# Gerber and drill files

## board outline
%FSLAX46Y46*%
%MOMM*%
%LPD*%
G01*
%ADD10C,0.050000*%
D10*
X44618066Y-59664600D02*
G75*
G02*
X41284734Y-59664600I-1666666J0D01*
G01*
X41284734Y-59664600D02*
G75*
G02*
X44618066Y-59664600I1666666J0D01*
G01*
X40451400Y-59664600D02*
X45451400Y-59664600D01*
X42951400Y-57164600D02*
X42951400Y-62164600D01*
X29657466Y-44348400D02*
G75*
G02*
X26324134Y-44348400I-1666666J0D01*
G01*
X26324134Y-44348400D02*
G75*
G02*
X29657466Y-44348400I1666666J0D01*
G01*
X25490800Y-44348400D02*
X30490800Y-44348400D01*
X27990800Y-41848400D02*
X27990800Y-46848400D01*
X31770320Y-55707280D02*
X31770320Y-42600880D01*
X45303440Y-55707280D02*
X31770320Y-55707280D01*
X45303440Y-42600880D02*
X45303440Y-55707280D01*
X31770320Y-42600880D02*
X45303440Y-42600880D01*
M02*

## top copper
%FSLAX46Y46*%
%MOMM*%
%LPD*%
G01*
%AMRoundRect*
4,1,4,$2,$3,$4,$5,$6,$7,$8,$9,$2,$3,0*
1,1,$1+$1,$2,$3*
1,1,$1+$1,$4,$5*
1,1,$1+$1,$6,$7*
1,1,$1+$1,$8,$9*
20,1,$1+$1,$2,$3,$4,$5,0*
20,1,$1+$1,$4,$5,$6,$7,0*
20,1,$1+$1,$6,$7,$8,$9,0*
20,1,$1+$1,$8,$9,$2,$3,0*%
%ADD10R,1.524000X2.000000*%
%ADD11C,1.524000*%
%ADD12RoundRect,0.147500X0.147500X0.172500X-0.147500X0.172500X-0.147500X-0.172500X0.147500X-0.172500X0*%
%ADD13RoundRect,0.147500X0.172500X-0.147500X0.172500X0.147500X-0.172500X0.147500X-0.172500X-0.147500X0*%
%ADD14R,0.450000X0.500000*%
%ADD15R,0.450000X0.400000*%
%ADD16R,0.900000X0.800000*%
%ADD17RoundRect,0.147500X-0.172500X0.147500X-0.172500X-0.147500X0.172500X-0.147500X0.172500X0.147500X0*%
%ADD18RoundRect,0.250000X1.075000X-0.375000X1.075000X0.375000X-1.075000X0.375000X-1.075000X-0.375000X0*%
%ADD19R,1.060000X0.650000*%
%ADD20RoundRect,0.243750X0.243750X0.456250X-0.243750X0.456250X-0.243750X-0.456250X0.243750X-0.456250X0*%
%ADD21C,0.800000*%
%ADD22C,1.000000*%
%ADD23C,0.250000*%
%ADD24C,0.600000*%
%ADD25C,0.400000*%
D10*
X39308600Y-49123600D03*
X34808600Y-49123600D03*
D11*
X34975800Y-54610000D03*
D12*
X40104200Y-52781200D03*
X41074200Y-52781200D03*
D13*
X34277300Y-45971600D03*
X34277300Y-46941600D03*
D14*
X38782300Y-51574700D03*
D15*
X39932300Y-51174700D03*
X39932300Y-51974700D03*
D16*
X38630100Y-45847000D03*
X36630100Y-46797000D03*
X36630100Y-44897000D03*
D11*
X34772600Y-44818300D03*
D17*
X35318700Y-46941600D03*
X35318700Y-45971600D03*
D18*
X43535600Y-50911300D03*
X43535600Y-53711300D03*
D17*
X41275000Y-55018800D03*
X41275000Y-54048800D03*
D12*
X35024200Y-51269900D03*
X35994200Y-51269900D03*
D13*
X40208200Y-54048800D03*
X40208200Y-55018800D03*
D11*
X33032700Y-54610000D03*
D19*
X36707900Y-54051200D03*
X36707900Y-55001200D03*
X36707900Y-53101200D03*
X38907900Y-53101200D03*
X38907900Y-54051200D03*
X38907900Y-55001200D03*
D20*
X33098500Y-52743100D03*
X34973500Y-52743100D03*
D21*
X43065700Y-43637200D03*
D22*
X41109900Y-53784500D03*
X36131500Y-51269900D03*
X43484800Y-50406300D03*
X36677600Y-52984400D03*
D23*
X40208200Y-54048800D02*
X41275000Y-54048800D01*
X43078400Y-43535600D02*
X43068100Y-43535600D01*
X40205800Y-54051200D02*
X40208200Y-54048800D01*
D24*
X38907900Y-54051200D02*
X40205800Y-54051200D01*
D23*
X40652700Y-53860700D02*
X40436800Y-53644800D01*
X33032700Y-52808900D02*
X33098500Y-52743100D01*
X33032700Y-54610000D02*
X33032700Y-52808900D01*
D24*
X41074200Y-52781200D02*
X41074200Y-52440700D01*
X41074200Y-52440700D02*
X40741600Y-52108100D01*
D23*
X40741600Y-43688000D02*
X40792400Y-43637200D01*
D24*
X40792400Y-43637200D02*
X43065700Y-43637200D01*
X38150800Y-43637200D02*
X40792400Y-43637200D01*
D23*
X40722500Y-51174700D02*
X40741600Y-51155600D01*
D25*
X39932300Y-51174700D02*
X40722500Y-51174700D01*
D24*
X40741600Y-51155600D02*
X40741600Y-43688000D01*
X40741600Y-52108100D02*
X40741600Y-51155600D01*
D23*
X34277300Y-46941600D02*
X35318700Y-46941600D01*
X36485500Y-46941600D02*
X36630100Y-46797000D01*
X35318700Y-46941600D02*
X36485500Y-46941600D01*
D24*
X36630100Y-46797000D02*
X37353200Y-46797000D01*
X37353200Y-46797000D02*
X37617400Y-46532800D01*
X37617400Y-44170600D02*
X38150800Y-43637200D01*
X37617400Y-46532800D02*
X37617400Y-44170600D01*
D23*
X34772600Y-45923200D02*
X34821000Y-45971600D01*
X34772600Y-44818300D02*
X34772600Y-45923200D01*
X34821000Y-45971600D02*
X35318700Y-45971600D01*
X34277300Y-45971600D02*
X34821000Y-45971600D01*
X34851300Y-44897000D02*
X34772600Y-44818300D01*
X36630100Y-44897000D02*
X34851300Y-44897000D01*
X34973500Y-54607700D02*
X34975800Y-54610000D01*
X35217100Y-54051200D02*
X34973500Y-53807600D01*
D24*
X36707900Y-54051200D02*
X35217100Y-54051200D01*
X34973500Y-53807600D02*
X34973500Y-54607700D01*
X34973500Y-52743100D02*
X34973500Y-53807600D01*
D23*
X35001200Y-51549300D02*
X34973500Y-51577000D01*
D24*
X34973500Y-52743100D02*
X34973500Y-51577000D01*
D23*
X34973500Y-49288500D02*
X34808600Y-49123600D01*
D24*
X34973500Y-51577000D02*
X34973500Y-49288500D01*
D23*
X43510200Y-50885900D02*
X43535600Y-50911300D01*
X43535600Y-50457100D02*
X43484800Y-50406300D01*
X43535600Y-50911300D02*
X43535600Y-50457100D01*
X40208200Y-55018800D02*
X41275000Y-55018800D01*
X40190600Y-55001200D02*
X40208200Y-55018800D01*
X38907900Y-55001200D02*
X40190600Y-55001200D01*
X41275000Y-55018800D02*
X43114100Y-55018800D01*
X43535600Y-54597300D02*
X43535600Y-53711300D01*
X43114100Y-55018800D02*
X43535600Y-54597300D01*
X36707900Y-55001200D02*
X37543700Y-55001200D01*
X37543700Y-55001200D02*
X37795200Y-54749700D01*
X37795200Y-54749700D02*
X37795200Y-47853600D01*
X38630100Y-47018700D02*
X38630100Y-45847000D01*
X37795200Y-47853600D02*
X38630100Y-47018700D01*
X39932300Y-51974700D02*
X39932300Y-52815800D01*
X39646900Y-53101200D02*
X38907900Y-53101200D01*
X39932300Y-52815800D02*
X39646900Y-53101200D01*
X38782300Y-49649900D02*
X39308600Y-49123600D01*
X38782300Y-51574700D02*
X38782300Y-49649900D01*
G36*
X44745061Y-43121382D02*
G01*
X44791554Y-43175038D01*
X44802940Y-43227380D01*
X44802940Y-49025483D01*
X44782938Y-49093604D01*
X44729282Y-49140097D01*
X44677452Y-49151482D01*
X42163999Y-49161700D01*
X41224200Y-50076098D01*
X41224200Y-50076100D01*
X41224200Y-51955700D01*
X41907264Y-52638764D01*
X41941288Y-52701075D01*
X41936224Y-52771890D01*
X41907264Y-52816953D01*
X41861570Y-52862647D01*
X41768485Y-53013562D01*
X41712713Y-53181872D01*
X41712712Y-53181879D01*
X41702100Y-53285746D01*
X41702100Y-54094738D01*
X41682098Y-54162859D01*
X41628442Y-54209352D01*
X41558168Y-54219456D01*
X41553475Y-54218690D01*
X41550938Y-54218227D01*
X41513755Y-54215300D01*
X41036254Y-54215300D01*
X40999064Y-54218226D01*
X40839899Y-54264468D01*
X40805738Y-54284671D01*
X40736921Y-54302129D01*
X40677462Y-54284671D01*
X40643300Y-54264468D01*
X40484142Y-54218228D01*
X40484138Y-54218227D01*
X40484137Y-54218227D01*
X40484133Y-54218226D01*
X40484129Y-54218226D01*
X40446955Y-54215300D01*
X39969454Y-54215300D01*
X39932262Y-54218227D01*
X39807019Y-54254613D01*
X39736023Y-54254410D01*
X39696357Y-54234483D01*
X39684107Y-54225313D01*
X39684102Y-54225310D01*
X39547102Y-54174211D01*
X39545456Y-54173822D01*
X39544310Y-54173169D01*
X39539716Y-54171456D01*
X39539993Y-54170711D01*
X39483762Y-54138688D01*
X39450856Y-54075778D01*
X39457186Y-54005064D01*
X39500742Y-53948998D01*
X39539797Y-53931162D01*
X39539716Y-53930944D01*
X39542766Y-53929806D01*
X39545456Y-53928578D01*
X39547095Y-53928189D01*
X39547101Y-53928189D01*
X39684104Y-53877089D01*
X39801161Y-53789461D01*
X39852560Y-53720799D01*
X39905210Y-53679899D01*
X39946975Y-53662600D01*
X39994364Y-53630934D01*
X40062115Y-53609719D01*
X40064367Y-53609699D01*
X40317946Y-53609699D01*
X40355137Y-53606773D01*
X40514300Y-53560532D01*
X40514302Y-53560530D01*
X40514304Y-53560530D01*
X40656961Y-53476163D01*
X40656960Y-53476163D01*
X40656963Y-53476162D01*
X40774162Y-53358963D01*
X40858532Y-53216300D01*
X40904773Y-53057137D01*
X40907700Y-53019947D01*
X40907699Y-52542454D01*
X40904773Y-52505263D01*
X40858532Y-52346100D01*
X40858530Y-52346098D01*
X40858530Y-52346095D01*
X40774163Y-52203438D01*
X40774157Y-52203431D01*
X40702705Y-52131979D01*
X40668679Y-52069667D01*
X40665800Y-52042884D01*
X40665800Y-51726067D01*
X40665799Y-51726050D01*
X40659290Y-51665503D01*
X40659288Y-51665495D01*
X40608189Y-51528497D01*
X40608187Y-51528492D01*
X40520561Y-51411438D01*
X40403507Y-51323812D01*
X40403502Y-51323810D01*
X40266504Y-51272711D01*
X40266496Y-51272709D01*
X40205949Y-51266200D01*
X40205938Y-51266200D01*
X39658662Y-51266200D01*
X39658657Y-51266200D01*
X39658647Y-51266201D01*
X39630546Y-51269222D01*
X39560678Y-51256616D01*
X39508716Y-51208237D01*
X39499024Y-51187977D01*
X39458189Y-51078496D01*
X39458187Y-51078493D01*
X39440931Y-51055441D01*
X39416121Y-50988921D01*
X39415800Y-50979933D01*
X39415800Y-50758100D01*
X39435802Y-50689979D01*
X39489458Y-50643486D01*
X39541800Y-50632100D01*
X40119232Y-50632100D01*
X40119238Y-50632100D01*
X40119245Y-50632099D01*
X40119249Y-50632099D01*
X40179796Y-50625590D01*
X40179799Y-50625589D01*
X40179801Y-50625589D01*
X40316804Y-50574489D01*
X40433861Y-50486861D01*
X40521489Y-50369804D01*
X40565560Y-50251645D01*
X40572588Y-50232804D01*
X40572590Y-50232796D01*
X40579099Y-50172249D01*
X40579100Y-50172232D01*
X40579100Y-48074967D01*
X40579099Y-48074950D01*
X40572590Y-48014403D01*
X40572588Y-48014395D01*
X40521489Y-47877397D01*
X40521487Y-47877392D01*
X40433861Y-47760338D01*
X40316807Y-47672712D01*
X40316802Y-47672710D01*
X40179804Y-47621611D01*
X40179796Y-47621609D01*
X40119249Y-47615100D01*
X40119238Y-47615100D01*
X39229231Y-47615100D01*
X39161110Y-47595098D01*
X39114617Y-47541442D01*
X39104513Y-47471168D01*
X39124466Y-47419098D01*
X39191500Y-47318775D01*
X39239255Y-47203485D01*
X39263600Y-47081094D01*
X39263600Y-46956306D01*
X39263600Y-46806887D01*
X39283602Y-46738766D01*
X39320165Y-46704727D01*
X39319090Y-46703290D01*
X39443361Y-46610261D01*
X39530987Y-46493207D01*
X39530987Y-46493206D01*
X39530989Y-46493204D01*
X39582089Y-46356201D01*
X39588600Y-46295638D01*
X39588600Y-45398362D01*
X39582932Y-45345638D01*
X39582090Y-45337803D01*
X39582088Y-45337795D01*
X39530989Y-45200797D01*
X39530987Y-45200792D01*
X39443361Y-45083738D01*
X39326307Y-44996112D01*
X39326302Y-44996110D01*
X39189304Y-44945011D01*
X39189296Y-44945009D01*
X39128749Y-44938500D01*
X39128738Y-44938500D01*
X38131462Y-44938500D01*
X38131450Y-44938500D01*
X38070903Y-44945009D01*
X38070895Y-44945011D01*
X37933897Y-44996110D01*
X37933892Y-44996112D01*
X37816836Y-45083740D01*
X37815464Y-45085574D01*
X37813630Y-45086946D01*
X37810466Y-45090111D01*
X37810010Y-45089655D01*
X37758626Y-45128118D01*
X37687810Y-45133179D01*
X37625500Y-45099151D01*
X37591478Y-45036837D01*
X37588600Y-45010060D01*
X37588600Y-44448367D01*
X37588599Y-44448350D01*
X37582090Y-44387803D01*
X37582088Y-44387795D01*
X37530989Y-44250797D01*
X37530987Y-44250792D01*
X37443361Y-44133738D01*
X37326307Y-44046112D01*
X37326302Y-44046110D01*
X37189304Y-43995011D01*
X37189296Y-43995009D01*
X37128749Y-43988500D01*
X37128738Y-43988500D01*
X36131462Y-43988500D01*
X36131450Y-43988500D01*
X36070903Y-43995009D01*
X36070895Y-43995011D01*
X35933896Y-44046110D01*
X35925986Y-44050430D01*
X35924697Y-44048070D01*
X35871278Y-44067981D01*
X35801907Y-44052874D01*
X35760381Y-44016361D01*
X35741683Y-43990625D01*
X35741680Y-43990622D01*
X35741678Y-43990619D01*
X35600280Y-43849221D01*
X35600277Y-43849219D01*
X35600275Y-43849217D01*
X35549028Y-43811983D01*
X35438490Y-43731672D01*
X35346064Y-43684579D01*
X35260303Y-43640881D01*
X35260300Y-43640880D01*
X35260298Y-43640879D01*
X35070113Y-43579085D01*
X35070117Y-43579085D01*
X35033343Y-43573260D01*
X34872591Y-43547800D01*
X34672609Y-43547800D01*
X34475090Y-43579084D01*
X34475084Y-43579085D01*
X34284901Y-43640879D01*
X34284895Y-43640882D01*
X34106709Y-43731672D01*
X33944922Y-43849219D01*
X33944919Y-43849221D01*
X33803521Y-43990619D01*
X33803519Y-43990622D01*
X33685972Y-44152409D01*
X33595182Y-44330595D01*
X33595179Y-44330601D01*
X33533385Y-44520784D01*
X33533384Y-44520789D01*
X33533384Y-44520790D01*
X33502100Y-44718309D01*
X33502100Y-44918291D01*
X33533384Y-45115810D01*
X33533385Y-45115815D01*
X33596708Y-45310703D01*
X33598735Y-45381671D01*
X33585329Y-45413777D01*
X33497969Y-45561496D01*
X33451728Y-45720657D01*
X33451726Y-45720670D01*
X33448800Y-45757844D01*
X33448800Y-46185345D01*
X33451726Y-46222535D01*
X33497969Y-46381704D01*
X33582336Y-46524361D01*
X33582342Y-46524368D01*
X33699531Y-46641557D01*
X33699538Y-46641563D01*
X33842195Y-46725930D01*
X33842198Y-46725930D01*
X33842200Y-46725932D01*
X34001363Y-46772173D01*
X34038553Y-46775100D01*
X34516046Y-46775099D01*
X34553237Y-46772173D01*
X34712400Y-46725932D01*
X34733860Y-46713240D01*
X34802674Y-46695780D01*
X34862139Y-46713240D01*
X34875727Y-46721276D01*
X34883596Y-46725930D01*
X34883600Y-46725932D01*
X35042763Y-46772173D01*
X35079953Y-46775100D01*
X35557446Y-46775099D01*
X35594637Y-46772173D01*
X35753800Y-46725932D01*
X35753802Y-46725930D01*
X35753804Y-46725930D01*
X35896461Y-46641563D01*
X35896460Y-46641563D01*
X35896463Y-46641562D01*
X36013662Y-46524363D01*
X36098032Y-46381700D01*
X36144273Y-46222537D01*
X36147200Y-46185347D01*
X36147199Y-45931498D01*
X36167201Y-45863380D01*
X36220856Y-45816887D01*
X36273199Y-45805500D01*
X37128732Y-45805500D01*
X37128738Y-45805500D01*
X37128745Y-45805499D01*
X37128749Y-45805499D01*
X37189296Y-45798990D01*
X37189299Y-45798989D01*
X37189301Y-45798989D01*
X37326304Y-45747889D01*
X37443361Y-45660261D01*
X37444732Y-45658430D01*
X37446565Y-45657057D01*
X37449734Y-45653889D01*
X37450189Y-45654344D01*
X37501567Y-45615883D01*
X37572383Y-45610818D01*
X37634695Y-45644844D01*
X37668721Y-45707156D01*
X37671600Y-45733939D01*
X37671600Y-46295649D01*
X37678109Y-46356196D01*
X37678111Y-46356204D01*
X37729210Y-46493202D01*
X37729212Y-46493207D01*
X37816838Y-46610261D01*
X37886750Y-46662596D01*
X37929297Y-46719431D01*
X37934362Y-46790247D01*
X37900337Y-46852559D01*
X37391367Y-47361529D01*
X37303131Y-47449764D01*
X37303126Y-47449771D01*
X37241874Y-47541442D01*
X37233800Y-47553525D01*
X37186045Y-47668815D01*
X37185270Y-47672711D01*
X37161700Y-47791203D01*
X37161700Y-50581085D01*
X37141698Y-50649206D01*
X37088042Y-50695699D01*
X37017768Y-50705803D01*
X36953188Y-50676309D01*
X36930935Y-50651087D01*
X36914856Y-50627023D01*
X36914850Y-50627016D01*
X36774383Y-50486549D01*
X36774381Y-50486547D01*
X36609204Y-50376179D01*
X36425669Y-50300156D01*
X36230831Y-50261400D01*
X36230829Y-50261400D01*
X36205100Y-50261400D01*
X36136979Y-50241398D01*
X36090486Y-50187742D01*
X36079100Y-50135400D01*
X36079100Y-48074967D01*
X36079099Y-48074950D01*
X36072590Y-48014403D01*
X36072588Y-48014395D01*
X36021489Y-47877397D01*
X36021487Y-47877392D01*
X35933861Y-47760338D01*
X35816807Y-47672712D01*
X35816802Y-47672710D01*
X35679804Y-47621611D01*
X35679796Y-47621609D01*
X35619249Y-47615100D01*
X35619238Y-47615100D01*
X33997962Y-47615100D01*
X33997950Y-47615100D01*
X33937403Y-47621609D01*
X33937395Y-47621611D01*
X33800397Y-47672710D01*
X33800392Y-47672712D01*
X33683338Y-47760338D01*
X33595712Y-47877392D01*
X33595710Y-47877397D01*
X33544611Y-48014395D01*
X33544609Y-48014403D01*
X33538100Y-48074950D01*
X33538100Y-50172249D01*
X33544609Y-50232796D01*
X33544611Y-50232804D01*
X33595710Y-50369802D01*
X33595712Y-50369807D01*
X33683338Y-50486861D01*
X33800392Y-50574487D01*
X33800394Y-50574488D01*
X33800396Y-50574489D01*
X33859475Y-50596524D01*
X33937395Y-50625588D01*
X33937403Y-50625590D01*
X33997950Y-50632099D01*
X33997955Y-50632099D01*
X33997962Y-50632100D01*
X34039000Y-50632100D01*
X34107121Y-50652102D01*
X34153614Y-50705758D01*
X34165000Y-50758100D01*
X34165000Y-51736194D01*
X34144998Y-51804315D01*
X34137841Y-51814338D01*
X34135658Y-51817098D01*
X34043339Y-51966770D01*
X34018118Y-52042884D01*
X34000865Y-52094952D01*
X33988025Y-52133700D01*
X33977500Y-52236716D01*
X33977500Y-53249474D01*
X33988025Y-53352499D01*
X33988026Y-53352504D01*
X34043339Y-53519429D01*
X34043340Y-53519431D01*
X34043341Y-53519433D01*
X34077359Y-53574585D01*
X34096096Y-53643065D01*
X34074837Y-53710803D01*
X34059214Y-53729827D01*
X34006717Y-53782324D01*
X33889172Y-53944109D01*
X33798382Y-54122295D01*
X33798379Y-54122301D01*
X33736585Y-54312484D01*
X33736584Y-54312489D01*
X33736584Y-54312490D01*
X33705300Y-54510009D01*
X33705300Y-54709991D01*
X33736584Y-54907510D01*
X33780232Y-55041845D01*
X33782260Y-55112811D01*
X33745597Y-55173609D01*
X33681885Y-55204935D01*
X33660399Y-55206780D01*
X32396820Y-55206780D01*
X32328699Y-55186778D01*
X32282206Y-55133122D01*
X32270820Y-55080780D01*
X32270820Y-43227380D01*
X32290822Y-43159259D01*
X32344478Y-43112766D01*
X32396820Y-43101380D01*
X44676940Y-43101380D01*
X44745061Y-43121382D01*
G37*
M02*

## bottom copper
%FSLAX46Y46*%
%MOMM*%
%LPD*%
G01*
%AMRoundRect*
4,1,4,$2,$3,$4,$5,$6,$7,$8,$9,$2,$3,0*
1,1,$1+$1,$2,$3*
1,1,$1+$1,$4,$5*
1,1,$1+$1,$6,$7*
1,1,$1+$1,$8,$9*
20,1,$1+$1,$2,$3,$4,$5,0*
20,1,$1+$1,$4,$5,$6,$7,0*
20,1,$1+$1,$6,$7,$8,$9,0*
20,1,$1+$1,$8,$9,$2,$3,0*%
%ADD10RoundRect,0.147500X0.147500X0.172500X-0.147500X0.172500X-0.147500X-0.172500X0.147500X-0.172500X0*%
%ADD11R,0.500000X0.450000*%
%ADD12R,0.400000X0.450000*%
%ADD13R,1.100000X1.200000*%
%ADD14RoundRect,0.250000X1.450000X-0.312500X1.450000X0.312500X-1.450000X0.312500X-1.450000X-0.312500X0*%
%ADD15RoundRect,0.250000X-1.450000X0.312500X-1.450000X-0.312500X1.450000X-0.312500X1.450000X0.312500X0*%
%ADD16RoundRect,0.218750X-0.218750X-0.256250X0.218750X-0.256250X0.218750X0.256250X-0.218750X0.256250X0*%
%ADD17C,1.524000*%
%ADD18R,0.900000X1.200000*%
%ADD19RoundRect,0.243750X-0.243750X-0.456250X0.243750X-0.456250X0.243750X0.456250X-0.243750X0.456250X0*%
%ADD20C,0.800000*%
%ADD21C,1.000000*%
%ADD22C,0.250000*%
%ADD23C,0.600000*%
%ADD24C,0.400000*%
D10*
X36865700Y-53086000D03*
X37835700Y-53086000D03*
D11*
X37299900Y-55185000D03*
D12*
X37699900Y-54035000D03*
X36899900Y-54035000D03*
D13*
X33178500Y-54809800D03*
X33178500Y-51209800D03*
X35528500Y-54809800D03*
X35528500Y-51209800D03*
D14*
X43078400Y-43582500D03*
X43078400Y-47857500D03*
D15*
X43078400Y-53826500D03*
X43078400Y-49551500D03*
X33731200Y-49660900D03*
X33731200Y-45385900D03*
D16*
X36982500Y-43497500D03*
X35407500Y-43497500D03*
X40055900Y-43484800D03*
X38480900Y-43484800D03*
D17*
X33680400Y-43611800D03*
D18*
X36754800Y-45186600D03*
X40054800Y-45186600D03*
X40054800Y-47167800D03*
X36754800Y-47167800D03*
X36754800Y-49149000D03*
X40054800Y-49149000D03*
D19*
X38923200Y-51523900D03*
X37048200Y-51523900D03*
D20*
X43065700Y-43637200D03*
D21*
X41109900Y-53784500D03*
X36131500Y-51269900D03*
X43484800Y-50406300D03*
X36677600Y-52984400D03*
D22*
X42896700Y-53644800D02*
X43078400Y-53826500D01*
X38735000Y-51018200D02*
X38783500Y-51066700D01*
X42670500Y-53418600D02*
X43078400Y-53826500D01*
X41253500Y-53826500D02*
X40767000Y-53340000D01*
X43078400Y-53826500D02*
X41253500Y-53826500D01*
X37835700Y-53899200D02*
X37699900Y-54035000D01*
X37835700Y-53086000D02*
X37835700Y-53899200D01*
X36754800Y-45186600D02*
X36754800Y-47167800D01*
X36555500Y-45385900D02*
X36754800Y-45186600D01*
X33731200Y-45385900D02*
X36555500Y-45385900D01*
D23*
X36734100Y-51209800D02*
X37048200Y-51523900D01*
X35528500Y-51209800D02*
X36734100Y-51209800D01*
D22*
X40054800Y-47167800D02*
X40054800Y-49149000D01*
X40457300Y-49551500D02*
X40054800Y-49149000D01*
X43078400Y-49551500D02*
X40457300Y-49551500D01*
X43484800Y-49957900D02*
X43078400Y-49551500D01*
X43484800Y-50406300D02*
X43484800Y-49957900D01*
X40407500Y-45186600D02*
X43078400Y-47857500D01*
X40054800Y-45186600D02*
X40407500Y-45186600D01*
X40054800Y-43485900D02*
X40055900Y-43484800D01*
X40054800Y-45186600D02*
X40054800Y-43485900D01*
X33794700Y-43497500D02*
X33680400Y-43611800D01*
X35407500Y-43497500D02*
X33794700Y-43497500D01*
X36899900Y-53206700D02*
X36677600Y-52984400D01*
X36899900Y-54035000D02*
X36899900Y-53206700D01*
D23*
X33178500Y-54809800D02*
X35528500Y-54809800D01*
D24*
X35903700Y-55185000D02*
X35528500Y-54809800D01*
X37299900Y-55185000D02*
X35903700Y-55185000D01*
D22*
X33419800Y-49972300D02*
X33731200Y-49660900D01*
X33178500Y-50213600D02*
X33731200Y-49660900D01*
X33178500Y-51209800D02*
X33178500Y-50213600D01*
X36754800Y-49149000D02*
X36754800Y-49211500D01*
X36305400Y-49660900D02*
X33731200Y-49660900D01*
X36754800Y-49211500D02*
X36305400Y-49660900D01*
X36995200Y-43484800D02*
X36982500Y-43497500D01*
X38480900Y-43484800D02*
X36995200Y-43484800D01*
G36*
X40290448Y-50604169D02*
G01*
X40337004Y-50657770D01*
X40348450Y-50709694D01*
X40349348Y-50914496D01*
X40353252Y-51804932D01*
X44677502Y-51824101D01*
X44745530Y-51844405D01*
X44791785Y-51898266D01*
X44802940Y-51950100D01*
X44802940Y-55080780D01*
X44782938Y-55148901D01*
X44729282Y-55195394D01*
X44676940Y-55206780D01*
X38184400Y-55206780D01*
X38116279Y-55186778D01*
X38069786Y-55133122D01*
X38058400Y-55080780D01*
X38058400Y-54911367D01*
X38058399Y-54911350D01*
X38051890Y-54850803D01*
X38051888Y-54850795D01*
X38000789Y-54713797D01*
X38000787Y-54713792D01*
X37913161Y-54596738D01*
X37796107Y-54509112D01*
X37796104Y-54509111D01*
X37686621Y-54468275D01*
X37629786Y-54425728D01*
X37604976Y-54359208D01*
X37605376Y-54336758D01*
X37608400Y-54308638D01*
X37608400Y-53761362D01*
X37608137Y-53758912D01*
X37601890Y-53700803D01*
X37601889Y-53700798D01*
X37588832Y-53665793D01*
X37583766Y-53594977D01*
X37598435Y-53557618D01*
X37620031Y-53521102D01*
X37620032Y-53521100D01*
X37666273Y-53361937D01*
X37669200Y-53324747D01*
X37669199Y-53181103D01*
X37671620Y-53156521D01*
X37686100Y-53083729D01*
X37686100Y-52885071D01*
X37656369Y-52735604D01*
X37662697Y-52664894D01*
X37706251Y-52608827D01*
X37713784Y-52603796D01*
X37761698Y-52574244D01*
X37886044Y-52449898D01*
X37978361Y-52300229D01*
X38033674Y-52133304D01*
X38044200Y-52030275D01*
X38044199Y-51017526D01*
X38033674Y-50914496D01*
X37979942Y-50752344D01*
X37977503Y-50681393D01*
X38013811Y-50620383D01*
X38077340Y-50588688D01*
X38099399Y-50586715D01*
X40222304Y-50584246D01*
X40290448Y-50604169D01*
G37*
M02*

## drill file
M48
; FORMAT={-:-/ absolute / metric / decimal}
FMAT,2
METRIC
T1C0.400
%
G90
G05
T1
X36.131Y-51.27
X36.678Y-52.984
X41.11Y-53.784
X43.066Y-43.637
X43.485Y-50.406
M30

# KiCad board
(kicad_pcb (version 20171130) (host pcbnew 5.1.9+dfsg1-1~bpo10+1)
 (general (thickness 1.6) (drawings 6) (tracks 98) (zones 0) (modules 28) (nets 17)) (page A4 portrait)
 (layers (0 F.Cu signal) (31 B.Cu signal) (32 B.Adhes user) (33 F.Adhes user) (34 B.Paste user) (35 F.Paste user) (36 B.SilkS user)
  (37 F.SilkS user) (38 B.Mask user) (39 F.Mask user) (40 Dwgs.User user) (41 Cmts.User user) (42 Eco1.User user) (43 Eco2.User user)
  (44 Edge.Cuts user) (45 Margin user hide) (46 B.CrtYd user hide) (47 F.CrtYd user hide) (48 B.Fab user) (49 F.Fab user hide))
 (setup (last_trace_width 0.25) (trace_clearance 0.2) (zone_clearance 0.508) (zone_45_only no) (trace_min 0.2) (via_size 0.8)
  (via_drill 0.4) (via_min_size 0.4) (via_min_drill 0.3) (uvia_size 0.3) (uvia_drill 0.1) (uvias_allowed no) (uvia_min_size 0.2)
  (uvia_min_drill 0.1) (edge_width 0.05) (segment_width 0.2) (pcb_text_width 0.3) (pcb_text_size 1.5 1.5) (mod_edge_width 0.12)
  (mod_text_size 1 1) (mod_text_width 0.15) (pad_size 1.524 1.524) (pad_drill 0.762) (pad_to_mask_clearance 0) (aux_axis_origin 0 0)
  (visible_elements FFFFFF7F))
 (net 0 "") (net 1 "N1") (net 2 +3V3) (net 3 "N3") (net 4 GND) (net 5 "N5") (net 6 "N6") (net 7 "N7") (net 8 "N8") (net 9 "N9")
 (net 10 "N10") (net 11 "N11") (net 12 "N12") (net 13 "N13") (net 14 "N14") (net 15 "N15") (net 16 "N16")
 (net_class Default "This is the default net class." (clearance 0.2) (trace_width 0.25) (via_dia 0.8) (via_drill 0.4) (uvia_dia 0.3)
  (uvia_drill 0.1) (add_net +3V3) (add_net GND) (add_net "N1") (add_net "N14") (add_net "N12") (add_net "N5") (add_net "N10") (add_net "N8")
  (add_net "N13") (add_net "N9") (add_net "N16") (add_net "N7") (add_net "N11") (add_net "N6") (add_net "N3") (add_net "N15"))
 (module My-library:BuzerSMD (layer F.Cu) (at 37.0586 49.1236 180)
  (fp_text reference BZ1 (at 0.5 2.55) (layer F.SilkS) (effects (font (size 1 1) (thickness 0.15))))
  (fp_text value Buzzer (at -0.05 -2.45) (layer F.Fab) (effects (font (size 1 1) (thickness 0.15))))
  (pad 2 smd rect (at -2.25 0 180) (size 1.524 2) (layers F.Cu F.Paste F.Mask) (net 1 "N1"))
  (pad 1 smd rect (at 2.25 0 180) (size 1.524 2) (layers F.Cu F.Paste F.Mask) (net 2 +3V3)))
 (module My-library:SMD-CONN (layer F.Cu) (at 34.9758 54.61)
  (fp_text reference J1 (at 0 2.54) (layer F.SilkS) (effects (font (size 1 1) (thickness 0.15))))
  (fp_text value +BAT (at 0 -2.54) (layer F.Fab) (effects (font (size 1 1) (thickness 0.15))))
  (pad 1 smd circle (at 0 0) (size 1.524 1.524) (layers F.Cu F.Paste F.Mask) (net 2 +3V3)))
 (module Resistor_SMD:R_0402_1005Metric (layer F.Cu) (at 40.5892 52.7812 180)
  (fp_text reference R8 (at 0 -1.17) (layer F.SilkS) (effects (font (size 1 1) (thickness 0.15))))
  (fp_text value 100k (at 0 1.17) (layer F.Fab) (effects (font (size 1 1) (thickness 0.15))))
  (pad 2 smd roundrect (at 0.485 0 180) (size 0.59 0.64) (layers F.Cu F.Paste F.Mask) (roundrect_rratio 0.25) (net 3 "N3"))
  (pad 1 smd roundrect (at -0.485 0 180) (size 0.59 0.64) (layers F.Cu F.Paste F.Mask) (roundrect_rratio 0.25) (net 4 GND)))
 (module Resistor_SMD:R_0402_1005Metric (layer F.Cu) (at 34.2773 46.4566 90)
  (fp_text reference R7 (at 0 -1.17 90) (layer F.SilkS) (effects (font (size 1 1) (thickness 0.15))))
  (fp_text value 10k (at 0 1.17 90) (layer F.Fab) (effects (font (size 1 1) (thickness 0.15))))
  (pad 2 smd roundrect (at 0.485 0 90) (size 0.59 0.64) (layers F.Cu F.Paste F.Mask) (roundrect_rratio 0.25) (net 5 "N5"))
  (pad 1 smd roundrect (at -0.485 0 90) (size 0.59 0.64) (layers F.Cu F.Paste F.Mask) (roundrect_rratio 0.25) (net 4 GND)))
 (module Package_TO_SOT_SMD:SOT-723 (layer F.Cu) (at 39.3573 51.5747 180)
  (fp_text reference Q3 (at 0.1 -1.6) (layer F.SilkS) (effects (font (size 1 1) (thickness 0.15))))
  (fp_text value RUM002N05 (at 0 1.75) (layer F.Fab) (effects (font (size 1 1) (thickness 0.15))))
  (pad 3 smd rect (at 0.575 0 180) (size 0.45 0.5) (layers F.Cu F.Paste F.Mask) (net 1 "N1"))
  (pad 2 smd rect (at -0.575 0.4 180) (size 0.45 0.4) (layers F.Cu F.Paste F.Mask) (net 4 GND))
  (pad 1 smd rect (at -0.575 -0.4 180) (size 0.45 0.4) (layers F.Cu F.Paste F.Mask) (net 3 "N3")))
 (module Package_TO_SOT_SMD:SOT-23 (layer F.Cu) (at 37.6301 45.847)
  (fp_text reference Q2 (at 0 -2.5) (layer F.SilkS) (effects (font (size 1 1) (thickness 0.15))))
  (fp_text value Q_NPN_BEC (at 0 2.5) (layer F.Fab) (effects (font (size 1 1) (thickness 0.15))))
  (pad 3 smd rect (at 1 0) (size 0.9 0.8) (layers F.Cu F.Paste F.Mask) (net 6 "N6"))
  (pad 2 smd rect (at -1 0.95) (size 0.9 0.8) (layers F.Cu F.Paste F.Mask) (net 4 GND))
  (pad 1 smd rect (at -1 -0.95) (size 0.9 0.8) (layers F.Cu F.Paste F.Mask) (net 5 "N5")))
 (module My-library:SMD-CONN (layer F.Cu) (at 34.7726 44.8183)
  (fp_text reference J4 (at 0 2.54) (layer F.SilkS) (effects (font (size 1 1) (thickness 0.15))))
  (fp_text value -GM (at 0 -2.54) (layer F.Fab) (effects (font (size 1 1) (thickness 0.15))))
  (pad 1 smd circle (at 0 0) (size 1.524 1.524) (layers F.Cu F.Paste F.Mask) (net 5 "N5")))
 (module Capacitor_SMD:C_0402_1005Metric (layer F.Cu) (at 35.3187 46.4566 270)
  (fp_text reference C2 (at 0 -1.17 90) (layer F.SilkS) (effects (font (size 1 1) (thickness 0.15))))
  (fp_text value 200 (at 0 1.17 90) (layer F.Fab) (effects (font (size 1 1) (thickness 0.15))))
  (pad 2 smd roundrect (at 0.485 0 270) (size 0.59 0.64) (layers F.Cu F.Paste F.Mask) (roundrect_rratio 0.25) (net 4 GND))
  (pad 1 smd roundrect (at -0.485 0 270) (size 0.59 0.64) (layers F.Cu F.Paste F.Mask) (roundrect_rratio 0.25) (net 5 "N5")))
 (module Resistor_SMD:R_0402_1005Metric (layer B.Cu) (at 37.3507 53.086 180)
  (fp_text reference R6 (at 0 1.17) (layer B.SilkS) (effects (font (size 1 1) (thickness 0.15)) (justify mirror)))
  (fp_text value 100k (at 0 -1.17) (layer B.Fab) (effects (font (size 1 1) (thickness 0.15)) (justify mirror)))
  (pad 2 smd roundrect (at 0.485 0 180) (size 0.59 0.64) (layers B.Cu B.Paste B.Mask) (roundrect_rratio 0.25) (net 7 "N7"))
  (pad 1 smd roundrect (at -0.485 0 180) (size 0.59 0.64) (layers B.Cu B.Paste B.Mask) (roundrect_rratio 0.25) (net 4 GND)))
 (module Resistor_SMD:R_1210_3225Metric (layer F.Cu) (at 43.5356 52.3113 90)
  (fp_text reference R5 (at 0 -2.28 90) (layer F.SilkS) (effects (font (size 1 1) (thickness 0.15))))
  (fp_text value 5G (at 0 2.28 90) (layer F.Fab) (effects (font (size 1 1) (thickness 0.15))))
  (pad 2 smd roundrect (at 1.4 0 90) (size 1.25 2.65) (layers F.Cu F.Paste F.Mask) (roundrect_rratio 0.2) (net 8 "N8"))
  (pad 1 smd roundrect (at -1.4 0 90) (size 1.25 2.65) (layers F.Cu F.Paste F.Mask) (roundrect_rratio 0.2) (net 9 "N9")))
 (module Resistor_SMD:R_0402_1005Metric (layer F.Cu) (at 41.275 54.5338 270)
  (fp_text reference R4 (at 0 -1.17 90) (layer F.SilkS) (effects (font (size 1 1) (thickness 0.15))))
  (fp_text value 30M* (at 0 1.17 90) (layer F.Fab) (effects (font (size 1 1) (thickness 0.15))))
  (pad 2 smd roundrect (at 0.485 0 270) (size 0.59 0.64) (layers F.Cu F.Paste F.Mask) (roundrect_rratio 0.25) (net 9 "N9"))
  (pad 1 smd roundrect (at -0.485 0 270) (size 0.59 0.64) (layers F.Cu F.Paste F.Mask) (roundrect_rratio 0.25) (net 4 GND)))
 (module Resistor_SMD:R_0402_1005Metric (layer F.Cu) (at 35.5092 51.2699 180)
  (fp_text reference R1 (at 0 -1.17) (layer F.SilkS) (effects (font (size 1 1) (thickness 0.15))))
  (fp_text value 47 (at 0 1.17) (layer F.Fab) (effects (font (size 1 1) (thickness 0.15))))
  (pad 2 smd roundrect (at 0.485 0 180) (size 0.59 0.64) (layers F.Cu F.Paste F.Mask) (roundrect_rratio 0.25) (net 2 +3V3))
  (pad 1 smd roundrect (at -0.485 0 180) (size 0.59 0.64) (layers F.Cu F.Paste F.Mask) (roundrect_rratio 0.25) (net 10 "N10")))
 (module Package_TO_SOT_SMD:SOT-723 (layer B.Cu) (at 37.2999 54.61 270)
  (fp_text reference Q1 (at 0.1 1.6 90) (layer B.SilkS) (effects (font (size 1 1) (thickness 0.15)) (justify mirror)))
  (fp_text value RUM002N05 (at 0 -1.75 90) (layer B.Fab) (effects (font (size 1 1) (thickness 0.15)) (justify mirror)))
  (pad 3 smd rect (at 0.575 0 270) (size 0.45 0.5) (layers B.Cu B.Paste B.Mask) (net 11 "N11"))
  (pad 2 smd rect (at -0.575 -0.4 270) (size 0.45 0.4) (layers B.Cu B.Paste B.Mask) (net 4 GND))
  (pad 1 smd rect (at -0.575 0.4 270) (size 0.45 0.4) (layers B.Cu B.Paste B.Mask) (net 7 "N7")))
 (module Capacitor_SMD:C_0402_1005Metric (layer F.Cu) (at 40.2082 54.5338 90)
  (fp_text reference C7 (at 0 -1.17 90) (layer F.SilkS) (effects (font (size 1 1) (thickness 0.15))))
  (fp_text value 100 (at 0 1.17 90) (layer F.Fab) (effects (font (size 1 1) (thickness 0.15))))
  (pad 2 smd roundrect (at 0.485 0 90) (size 0.59 0.64) (layers F.Cu F.Paste F.Mask) (roundrect_rratio 0.25) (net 4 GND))
  (pad 1 smd roundrect (at -0.485 0 90) (size 0.59 0.64) (layers F.Cu F.Paste F.Mask) (roundrect_rratio 0.25) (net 9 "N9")))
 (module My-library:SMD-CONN (layer F.Cu) (at 33.0327 54.61)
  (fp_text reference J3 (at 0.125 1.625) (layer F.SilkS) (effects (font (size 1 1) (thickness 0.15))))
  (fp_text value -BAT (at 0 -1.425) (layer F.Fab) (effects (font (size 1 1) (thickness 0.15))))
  (pad 1 smd circle (at 0 0) (size 1.524 1.524) (layers F.Cu F.Paste F.Mask) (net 4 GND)))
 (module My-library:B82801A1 (layer B.Cu) (at 34.3535 53.0098)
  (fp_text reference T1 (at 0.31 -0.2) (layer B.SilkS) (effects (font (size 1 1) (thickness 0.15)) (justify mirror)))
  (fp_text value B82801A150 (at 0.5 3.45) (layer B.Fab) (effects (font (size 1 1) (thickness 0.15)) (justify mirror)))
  (pad 2 smd rect (at -1.175 1.8) (size 1.1 1.2) (layers B.Cu B.Paste B.Mask) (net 11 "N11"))
  (pad 1 smd rect (at -1.175 -1.8) (size 1.1 1.2) (layers B.Cu B.Paste B.Mask) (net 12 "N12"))
  (pad 3 smd rect (at 1.175 1.8) (size 1.1 1.2) (layers B.Cu B.Paste B.Mask) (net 11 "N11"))
  (pad 4 smd rect (at 1.175 -1.8) (size 1.1 1.2) (layers B.Cu B.Paste B.Mask) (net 10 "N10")))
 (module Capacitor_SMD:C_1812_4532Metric (layer B.Cu) (at 43.0784 45.72 90)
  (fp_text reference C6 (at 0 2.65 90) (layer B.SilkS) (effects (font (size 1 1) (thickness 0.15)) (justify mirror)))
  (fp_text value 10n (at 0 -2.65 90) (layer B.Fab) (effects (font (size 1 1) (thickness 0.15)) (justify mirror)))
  (pad 2 smd roundrect (at 2.1375 0 90) (size 1.125 3.4) (layers B.Cu B.Paste B.Mask) (roundrect_rratio 0.222222) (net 4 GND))
  (pad 1 smd roundrect (at -2.1375 0 90) (size 1.125 3.4) (layers B.Cu B.Paste B.Mask) (roundrect_rratio 0.222222) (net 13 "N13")))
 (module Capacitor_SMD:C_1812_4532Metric (layer B.Cu) (at 43.0784 51.689 270)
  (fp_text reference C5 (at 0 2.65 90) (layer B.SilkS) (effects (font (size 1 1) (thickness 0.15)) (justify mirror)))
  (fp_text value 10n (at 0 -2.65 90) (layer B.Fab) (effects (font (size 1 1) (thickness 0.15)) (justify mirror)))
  (pad 2 smd roundrect (at 2.1375 0 270) (size 1.125 3.4) (layers B.Cu B.Paste B.Mask) (roundrect_rratio 0.222222) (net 4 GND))
  (pad 1 smd roundrect (at -2.1375 0 270) (size 1.125 3.4) (layers B.Cu B.Paste B.Mask) (roundrect_rratio 0.222222) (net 8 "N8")))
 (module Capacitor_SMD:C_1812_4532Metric (layer B.Cu) (at 33.7312 47.5234 270)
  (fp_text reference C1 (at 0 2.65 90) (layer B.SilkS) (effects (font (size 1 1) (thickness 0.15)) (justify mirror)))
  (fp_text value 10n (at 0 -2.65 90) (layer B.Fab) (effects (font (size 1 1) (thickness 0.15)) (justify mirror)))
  (pad 2 smd roundrect (at 2.1375 0 270) (size 1.125 3.4) (layers B.Cu B.Paste B.Mask) (roundrect_rratio 0.222222) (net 12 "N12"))
  (pad 1 smd roundrect (at -2.1375 0 270) (size 1.125 3.4) (layers B.Cu B.Paste B.Mask) (roundrect_rratio 0.222222) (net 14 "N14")))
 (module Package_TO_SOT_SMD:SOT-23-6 (layer F.Cu) (at 37.8079 54.0512 180)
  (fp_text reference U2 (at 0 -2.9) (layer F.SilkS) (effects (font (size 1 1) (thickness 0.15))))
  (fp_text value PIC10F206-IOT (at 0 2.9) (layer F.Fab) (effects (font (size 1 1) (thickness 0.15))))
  (pad 5 smd rect (at 1.1 0 180) (size 1.06 0.65) (layers F.Cu F.Paste F.Mask) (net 2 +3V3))
  (pad 6 smd rect (at 1.1 -0.95 180) (size 1.06 0.65) (layers F.Cu F.Paste F.Mask) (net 6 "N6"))
  (pad 4 smd rect (at 1.1 0.95 180) (size 1.06 0.65) (layers F.Cu F.Paste F.Mask) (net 7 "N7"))
  (pad 3 smd rect (at -1.1 0.95 180) (size 1.06 0.65) (layers F.Cu F.Paste F.Mask) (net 3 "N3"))
  (pad 2 smd rect (at -1.1 0 180) (size 1.06 0.65) (layers F.Cu F.Paste F.Mask) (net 4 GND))
  (pad 1 smd rect (at -1.1 -0.95 180) (size 1.06 0.65) (layers F.Cu F.Paste F.Mask) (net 9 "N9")))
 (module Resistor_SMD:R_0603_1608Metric (layer B.Cu) (at 36.195 43.4975)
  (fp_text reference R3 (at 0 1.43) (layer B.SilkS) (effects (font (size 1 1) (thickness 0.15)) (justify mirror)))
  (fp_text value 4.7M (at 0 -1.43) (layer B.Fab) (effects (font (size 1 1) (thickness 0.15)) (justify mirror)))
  (pad 2 smd roundrect (at 0.7875 0) (size 0.875 0.95) (layers B.Cu B.Paste B.Mask) (roundrect_rratio 0.25) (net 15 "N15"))
  (pad 1 smd roundrect (at -0.7875 0) (size 0.875 0.95) (layers B.Cu B.Paste B.Mask) (roundrect_rratio 0.25) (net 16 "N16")))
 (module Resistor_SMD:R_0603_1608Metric (layer B.Cu) (at 39.2684 43.4848)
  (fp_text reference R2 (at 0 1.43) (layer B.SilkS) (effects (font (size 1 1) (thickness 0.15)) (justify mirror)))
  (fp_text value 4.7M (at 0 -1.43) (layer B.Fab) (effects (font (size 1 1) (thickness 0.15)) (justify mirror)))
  (pad 2 smd roundrect (at 0.7875 0) (size 0.875 0.95) (layers B.Cu B.Paste B.Mask) (roundrect_rratio 0.25) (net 13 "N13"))
  (pad 1 smd roundrect (at -0.7875 0) (size 0.875 0.95) (layers B.Cu B.Paste B.Mask) (roundrect_rratio 0.25) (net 15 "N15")))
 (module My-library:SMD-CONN (layer B.Cu) (at 33.6804 43.6118)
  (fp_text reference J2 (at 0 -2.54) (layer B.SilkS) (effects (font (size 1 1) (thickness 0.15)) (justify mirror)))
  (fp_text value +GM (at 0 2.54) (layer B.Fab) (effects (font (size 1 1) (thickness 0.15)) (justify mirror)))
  (pad 1 smd circle (at 0 0) (size 1.524 1.524) (layers B.Cu B.Paste B.Mask) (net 16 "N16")))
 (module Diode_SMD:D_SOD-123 (layer B.Cu) (at 38.4048 45.1866 180)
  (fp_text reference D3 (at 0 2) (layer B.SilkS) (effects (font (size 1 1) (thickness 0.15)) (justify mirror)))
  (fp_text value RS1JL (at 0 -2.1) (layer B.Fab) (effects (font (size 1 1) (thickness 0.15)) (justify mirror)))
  (pad 2 smd rect (at 1.65 0 180) (size 0.9 1.2) (layers B.Cu B.Paste B.Mask) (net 14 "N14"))
  (pad 1 smd rect (at -1.65 0 180) (size 0.9 1.2) (layers B.Cu B.Paste B.Mask) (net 13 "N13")))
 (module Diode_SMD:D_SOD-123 (layer B.Cu) (at 38.4048 47.1678)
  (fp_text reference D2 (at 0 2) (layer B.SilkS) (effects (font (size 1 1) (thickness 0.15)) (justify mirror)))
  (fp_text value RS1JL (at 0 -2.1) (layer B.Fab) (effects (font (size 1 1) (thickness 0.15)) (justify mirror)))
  (pad 2 smd rect (at 1.65 0) (size 0.9 1.2) (layers B.Cu B.Paste B.Mask) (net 8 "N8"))
  (pad 1 smd rect (at -1.65 0) (size 0.9 1.2) (layers B.Cu B.Paste B.Mask) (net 14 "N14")))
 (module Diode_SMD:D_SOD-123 (layer B.Cu) (at 38.4048 49.149 180)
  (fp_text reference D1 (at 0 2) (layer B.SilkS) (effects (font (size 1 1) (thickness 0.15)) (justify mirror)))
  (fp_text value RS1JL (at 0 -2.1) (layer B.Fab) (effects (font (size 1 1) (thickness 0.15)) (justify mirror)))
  (pad 2 smd rect (at 1.65 0 180) (size 0.9 1.2) (layers B.Cu B.Paste B.Mask) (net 12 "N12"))
  (pad 1 smd rect (at -1.65 0 180) (size 0.9 1.2) (layers B.Cu B.Paste B.Mask) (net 8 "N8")))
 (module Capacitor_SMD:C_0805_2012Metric (layer B.Cu) (at 37.9857 51.5239)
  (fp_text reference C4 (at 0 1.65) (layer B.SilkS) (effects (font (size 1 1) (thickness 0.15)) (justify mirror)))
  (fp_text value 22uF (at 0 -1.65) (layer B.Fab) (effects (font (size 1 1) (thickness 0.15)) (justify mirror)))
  (pad 2 smd roundrect (at 0.9375 0) (size 0.975 1.4) (layers B.Cu B.Paste B.Mask) (roundrect_rratio 0.25) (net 4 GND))
  (pad 1 smd roundrect (at -0.9375 0) (size 0.975 1.4) (layers B.Cu B.Paste B.Mask) (roundrect_rratio 0.25) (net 10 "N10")))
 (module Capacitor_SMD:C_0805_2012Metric (layer F.Cu) (at 34.036 52.7431 180)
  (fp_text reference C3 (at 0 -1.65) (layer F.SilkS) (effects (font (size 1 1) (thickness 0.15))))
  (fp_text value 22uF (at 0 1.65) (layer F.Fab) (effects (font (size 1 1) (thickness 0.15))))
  (pad 2 smd roundrect (at 0.9375 0 180) (size 0.975 1.4) (layers F.Cu F.Paste F.Mask) (roundrect_rratio 0.25) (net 4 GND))
  (pad 1 smd roundrect (at -0.9375 0 180) (size 0.975 1.4) (layers F.Cu F.Paste F.Mask) (roundrect_rratio 0.25) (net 2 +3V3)))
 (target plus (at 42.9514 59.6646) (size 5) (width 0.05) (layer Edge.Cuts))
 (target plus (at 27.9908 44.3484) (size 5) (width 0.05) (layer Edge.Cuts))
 (gr_line (start 31.77032 55.70728) (end 31.77032 42.60088) (layer Edge.Cuts) (width 0.05))
 (gr_line (start 45.30344 55.70728) (end 31.77032 55.70728) (layer Edge.Cuts) (width 0.05))
 (gr_line (start 45.30344 42.60088) (end 45.30344 55.70728) (layer Edge.Cuts) (width 0.05))
 (gr_line (start 31.77032 42.60088) (end 45.30344 42.60088) (layer Edge.Cuts) (width 0.05))
 (via (at 43.0657 43.6372) (size 0.8) (drill 0.4) (layers F.Cu B.Cu) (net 4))
 (segment (start 42.8967 53.6448) (end 43.0784 53.8265) (width 0.25) (layer B.Cu) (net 4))
 (segment (start 38.735 51.0182) (end 38.7835 51.0667) (width 0.25) (layer B.Cu) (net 4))
 (segment (start 42.6705 53.4186) (end 43.0784 53.8265) (width 0.25) (layer B.Cu) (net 4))
 (segment (start 40.2082 54.0488) (end 41.275 54.0488) (width 0.25) (layer F.Cu) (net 4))
 (segment (start 41.2535 53.8265) (end 40.767 53.34) (width 0.25) (layer B.Cu) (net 4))
 (segment (start 43.0784 53.8265) (end 41.2535 53.8265) (width 0.25) (layer B.Cu) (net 4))
 (segment (start 43.0784 43.5356) (end 43.0681 43.5356) (width 0.25) (layer F.Cu) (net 4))
 (segment (start 40.2058 54.0512) (end 40.2082 54.0488) (width 0.25) (layer F.Cu) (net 4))
 (segment (start 38.9079 54.0512) (end 40.2058 54.0512) (width 0.6) (layer F.Cu) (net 4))
 (segment (start 37.8357 53.8992) (end 37.6999 54.035) (width 0.25) (layer B.Cu) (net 4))
 (segment (start 37.8357 53.086) (end 37.8357 53.8992) (width 0.25) (layer B.Cu) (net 4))
 (segment (start 40.6527 53.8607) (end 40.4368 53.6448) (width 0.25) (layer F.Cu) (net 4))
 (via (at 41.1099 53.7845) (size 1) (drill 0.4) (layers F.Cu B.Cu) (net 4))
 (segment (start 33.0327 52.8089) (end 33.0985 52.7431) (width 0.25) (layer F.Cu) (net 4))
 (segment (start 33.0327 54.61) (end 33.0327 52.8089) (width 0.25) (layer F.Cu) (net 4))
 (segment (start 41.0742 52.7812) (end 41.0742 52.4407) (width 0.6) (layer F.Cu) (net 4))
 (segment (start 41.0742 52.4407) (end 40.7416 52.1081) (width 0.6) (layer F.Cu) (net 4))
 (segment (start 40.7416 43.688) (end 40.7924 43.6372) (width 0.25) (layer F.Cu) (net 4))
 (segment (start 40.7924 43.6372) (end 43.0657 43.6372) (width 0.6) (layer F.Cu) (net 4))
 (segment (start 38.1508 43.6372) (end 40.7924 43.6372) (width 0.6) (layer F.Cu) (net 4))
 (segment (start 40.7225 51.1747) (end 40.7416 51.1556) (width 0.25) (layer F.Cu) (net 4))
 (segment (start 39.9323 51.1747) (end 40.7225 51.1747) (width 0.4) (layer F.Cu) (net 4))
 (segment (start 40.7416 51.1556) (end 40.7416 43.688) (width 0.6) (layer F.Cu) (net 4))
 (segment (start 40.7416 52.1081) (end 40.7416 51.1556) (width 0.6) (layer F.Cu) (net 4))
 (segment (start 34.2773 46.9416) (end 35.3187 46.9416) (width 0.25) (layer F.Cu) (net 4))
 (segment (start 36.4855 46.9416) (end 36.6301 46.797) (width 0.25) (layer F.Cu) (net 4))
 (segment (start 35.3187 46.9416) (end 36.4855 46.9416) (width 0.25) (layer F.Cu) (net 4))
 (segment (start 36.6301 46.797) (end 37.3532 46.797) (width 0.6) (layer F.Cu) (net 4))
 (segment (start 37.3532 46.797) (end 37.6174 46.5328) (width 0.6) (layer F.Cu) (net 4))
 (segment (start 37.6174 44.1706) (end 38.1508 43.6372) (width 0.6) (layer F.Cu) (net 4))
 (segment (start 37.6174 46.5328) (end 37.6174 44.1706) (width 0.6) (layer F.Cu) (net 4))
 (segment (start 36.7548 45.1866) (end 36.7548 47.1678) (width 0.25) (layer B.Cu) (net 14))
 (segment (start 36.5555 45.3859) (end 36.7548 45.1866) (width 0.25) (layer B.Cu) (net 14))
 (segment (start 33.7312 45.3859) (end 36.5555 45.3859) (width 0.25) (layer B.Cu) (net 14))
 (segment (start 34.7726 45.9232) (end 34.821 45.9716) (width 0.25) (layer F.Cu) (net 5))
 (segment (start 34.7726 44.8183) (end 34.7726 45.9232) (width 0.25) (layer F.Cu) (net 5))
 (segment (start 34.821 45.9716) (end 35.3187 45.9716) (width 0.25) (layer F.Cu) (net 5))
 (segment (start 34.2773 45.9716) (end 34.821 45.9716) (width 0.25) (layer F.Cu) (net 5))
 (segment (start 34.8513 44.897) (end 34.7726 44.8183) (width 0.25) (layer F.Cu) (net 5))
 (segment (start 36.6301 44.897) (end 34.8513 44.897) (width 0.25) (layer F.Cu) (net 5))
 (segment (start 34.9735 54.6077) (end 34.9758 54.61) (width 0.25) (layer F.Cu) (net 2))
 (segment (start 35.2171 54.0512) (end 34.9735 53.8076) (width 0.25) (layer F.Cu) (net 2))
 (segment (start 36.7079 54.0512) (end 35.2171 54.0512) (width 0.6) (layer F.Cu) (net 2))
 (segment (start 34.9735 53.8076) (end 34.9735 54.6077) (width 0.6) (layer F.Cu) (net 2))
 (segment (start 34.9735 52.7431) (end 34.9735 53.8076) (width 0.6) (layer F.Cu) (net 2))
 (segment (start 35.0012 51.5493) (end 34.9735 51.577) (width 0.25) (layer F.Cu) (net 2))
 (segment (start 34.9735 52.7431) (end 34.9735 51.577) (width 0.6) (layer F.Cu) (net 2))
 (segment (start 34.9735 49.2885) (end 34.8086 49.1236) (width 0.25) (layer F.Cu) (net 2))
 (segment (start 34.9735 51.577) (end 34.9735 49.2885) (width 0.6) (layer F.Cu) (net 2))
 (via (at 36.1315 51.2699) (size 1) (drill 0.4) (layers F.Cu B.Cu) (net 10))
 (segment (start 36.7341 51.2098) (end 37.0482 51.5239) (width 0.6) (layer B.Cu) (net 10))
 (segment (start 35.5285 51.2098) (end 36.7341 51.2098) (width 0.6) (layer B.Cu) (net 10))
 (via (at 43.4848 50.4063) (size 1) (drill 0.4) (layers F.Cu B.Cu) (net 8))
 (segment (start 40.0548 47.1678) (end 40.0548 49.149) (width 0.25) (layer B.Cu) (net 8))
 (segment (start 40.4573 49.5515) (end 40.0548 49.149) (width 0.25) (layer B.Cu) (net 8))
 (segment (start 43.0784 49.5515) (end 40.4573 49.5515) (width 0.25) (layer B.Cu) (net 8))
 (segment (start 43.5102 50.8859) (end 43.5356 50.9113) (width 0.25) (layer F.Cu) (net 8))
 (segment (start 43.4848 49.9579) (end 43.0784 49.5515) (width 0.25) (layer B.Cu) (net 8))
 (segment (start 43.4848 50.4063) (end 43.4848 49.9579) (width 0.25) (layer B.Cu) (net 8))
 (segment (start 43.5356 50.4571) (end 43.4848 50.4063) (width 0.25) (layer F.Cu) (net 8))
 (segment (start 43.5356 50.9113) (end 43.5356 50.4571) (width 0.25) (layer F.Cu) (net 8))
 (segment (start 40.4075 45.1866) (end 43.0784 47.8575) (width 0.25) (layer B.Cu) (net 13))
 (segment (start 40.0548 45.1866) (end 40.4075 45.1866) (width 0.25) (layer B.Cu) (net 13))
 (segment (start 40.0548 43.4859) (end 40.0559 43.4848) (width 0.25) (layer B.Cu) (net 13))
 (segment (start 40.0548 45.1866) (end 40.0548 43.4859) (width 0.25) (layer B.Cu) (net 13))
 (segment (start 40.2082 55.0188) (end 41.275 55.0188) (width 0.25) (layer F.Cu) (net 9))
 (segment (start 40.1906 55.0012) (end 40.2082 55.0188) (width 0.25) (layer F.Cu) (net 9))
 (segment (start 38.9079 55.0012) (end 40.1906 55.0012) (width 0.25) (layer F.Cu) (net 9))
 (segment (start 41.275 55.0188) (end 43.1141 55.0188) (width 0.25) (layer F.Cu) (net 9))
 (segment (start 43.5356 54.5973) (end 43.5356 53.7113) (width 0.25) (layer F.Cu) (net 9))
 (segment (start 43.1141 55.0188) (end 43.5356 54.5973) (width 0.25) (layer F.Cu) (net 9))
 (segment (start 33.7947 43.4975) (end 33.6804 43.6118) (width 0.25) (layer B.Cu) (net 16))
 (segment (start 35.4075 43.4975) (end 33.7947 43.4975) (width 0.25) (layer B.Cu) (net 16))
 (via (at 36.6776 52.9844) (size 1) (drill 0.4) (layers F.Cu B.Cu) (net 7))
 (segment (start 36.8999 53.2067) (end 36.6776 52.9844) (width 0.25) (layer B.Cu) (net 7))
 (segment (start 36.8999 54.035) (end 36.8999 53.2067) (width 0.25) (layer B.Cu) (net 7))
 (segment (start 33.1785 54.8098) (end 35.5285 54.8098) (width 0.6) (layer B.Cu) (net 11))
 (segment (start 35.9037 55.185) (end 35.5285 54.8098) (width 0.4) (layer B.Cu) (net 11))
 (segment (start 37.2999 55.185) (end 35.9037 55.185) (width 0.4) (layer B.Cu) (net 11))
 (segment (start 33.4198 49.9723) (end 33.7312 49.6609) (width 0.25) (layer B.Cu) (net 12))
 (segment (start 33.1785 50.2136) (end 33.7312 49.6609) (width 0.25) (layer B.Cu) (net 12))
 (segment (start 33.1785 51.2098) (end 33.1785 50.2136) (width 0.25) (layer B.Cu) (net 12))
 (segment (start 36.7548 49.149) (end 36.7548 49.2115) (width 0.25) (layer B.Cu) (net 12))
 (segment (start 36.3054 49.6609) (end 33.7312 49.6609) (width 0.25) (layer B.Cu) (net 12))
 (segment (start 36.7548 49.2115) (end 36.3054 49.6609) (width 0.25) (layer B.Cu) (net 12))
 (segment (start 36.9952 43.4848) (end 36.9825 43.4975) (width 0.25) (layer B.Cu) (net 15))
 (segment (start 38.4809 43.4848) (end 36.9952 43.4848) (width 0.25) (layer B.Cu) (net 15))
 (segment (start 36.7079 55.0012) (end 37.5437 55.0012) (width 0.25) (layer F.Cu) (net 6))
 (segment (start 37.5437 55.0012) (end 37.7952 54.7497) (width 0.25) (layer F.Cu) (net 6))
 (segment (start 37.7952 54.7497) (end 37.7952 47.8536) (width 0.25) (layer F.Cu) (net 6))
 (segment (start 38.6301 47.0187) (end 38.6301 45.847) (width 0.25) (layer F.Cu) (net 6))
 (segment (start 37.7952 47.8536) (end 38.6301 47.0187) (width 0.25) (layer F.Cu) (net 6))
 (segment (start 39.9323 51.9747) (end 39.9323 52.8158) (width 0.25) (layer F.Cu) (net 3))
 (segment (start 39.6469 53.1012) (end 38.9079 53.1012) (width 0.25) (layer F.Cu) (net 3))
 (segment (start 39.9323 52.8158) (end 39.6469 53.1012) (width 0.25) (layer F.Cu) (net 3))
 (segment (start 38.7823 49.6499) (end 39.3086 49.1236) (width 0.25) (layer F.Cu) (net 1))
 (segment (start 38.7823 51.5747) (end 38.7823 49.6499) (width 0.25) (layer F.Cu) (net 1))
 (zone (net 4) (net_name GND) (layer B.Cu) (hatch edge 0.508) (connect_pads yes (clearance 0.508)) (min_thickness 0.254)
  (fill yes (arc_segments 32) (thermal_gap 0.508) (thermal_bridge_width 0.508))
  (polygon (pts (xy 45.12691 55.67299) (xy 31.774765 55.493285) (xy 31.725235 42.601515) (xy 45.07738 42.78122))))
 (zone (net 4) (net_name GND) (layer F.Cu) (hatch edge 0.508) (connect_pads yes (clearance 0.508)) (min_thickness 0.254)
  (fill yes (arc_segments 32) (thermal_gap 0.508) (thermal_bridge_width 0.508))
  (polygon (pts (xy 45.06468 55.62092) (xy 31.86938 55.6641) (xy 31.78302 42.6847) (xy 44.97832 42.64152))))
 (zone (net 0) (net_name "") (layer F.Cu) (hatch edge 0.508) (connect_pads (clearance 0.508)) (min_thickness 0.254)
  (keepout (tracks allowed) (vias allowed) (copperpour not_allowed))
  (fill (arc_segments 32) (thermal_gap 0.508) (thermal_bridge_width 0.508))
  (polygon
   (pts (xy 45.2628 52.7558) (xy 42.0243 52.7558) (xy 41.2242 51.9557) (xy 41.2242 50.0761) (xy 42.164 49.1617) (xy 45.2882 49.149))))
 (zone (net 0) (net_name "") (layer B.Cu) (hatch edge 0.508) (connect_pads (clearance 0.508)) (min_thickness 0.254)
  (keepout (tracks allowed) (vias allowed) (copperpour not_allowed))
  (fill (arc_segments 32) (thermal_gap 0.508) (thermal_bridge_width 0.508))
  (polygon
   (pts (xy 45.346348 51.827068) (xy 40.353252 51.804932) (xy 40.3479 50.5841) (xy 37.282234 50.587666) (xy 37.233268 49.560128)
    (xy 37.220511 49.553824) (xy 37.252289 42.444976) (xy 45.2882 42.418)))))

